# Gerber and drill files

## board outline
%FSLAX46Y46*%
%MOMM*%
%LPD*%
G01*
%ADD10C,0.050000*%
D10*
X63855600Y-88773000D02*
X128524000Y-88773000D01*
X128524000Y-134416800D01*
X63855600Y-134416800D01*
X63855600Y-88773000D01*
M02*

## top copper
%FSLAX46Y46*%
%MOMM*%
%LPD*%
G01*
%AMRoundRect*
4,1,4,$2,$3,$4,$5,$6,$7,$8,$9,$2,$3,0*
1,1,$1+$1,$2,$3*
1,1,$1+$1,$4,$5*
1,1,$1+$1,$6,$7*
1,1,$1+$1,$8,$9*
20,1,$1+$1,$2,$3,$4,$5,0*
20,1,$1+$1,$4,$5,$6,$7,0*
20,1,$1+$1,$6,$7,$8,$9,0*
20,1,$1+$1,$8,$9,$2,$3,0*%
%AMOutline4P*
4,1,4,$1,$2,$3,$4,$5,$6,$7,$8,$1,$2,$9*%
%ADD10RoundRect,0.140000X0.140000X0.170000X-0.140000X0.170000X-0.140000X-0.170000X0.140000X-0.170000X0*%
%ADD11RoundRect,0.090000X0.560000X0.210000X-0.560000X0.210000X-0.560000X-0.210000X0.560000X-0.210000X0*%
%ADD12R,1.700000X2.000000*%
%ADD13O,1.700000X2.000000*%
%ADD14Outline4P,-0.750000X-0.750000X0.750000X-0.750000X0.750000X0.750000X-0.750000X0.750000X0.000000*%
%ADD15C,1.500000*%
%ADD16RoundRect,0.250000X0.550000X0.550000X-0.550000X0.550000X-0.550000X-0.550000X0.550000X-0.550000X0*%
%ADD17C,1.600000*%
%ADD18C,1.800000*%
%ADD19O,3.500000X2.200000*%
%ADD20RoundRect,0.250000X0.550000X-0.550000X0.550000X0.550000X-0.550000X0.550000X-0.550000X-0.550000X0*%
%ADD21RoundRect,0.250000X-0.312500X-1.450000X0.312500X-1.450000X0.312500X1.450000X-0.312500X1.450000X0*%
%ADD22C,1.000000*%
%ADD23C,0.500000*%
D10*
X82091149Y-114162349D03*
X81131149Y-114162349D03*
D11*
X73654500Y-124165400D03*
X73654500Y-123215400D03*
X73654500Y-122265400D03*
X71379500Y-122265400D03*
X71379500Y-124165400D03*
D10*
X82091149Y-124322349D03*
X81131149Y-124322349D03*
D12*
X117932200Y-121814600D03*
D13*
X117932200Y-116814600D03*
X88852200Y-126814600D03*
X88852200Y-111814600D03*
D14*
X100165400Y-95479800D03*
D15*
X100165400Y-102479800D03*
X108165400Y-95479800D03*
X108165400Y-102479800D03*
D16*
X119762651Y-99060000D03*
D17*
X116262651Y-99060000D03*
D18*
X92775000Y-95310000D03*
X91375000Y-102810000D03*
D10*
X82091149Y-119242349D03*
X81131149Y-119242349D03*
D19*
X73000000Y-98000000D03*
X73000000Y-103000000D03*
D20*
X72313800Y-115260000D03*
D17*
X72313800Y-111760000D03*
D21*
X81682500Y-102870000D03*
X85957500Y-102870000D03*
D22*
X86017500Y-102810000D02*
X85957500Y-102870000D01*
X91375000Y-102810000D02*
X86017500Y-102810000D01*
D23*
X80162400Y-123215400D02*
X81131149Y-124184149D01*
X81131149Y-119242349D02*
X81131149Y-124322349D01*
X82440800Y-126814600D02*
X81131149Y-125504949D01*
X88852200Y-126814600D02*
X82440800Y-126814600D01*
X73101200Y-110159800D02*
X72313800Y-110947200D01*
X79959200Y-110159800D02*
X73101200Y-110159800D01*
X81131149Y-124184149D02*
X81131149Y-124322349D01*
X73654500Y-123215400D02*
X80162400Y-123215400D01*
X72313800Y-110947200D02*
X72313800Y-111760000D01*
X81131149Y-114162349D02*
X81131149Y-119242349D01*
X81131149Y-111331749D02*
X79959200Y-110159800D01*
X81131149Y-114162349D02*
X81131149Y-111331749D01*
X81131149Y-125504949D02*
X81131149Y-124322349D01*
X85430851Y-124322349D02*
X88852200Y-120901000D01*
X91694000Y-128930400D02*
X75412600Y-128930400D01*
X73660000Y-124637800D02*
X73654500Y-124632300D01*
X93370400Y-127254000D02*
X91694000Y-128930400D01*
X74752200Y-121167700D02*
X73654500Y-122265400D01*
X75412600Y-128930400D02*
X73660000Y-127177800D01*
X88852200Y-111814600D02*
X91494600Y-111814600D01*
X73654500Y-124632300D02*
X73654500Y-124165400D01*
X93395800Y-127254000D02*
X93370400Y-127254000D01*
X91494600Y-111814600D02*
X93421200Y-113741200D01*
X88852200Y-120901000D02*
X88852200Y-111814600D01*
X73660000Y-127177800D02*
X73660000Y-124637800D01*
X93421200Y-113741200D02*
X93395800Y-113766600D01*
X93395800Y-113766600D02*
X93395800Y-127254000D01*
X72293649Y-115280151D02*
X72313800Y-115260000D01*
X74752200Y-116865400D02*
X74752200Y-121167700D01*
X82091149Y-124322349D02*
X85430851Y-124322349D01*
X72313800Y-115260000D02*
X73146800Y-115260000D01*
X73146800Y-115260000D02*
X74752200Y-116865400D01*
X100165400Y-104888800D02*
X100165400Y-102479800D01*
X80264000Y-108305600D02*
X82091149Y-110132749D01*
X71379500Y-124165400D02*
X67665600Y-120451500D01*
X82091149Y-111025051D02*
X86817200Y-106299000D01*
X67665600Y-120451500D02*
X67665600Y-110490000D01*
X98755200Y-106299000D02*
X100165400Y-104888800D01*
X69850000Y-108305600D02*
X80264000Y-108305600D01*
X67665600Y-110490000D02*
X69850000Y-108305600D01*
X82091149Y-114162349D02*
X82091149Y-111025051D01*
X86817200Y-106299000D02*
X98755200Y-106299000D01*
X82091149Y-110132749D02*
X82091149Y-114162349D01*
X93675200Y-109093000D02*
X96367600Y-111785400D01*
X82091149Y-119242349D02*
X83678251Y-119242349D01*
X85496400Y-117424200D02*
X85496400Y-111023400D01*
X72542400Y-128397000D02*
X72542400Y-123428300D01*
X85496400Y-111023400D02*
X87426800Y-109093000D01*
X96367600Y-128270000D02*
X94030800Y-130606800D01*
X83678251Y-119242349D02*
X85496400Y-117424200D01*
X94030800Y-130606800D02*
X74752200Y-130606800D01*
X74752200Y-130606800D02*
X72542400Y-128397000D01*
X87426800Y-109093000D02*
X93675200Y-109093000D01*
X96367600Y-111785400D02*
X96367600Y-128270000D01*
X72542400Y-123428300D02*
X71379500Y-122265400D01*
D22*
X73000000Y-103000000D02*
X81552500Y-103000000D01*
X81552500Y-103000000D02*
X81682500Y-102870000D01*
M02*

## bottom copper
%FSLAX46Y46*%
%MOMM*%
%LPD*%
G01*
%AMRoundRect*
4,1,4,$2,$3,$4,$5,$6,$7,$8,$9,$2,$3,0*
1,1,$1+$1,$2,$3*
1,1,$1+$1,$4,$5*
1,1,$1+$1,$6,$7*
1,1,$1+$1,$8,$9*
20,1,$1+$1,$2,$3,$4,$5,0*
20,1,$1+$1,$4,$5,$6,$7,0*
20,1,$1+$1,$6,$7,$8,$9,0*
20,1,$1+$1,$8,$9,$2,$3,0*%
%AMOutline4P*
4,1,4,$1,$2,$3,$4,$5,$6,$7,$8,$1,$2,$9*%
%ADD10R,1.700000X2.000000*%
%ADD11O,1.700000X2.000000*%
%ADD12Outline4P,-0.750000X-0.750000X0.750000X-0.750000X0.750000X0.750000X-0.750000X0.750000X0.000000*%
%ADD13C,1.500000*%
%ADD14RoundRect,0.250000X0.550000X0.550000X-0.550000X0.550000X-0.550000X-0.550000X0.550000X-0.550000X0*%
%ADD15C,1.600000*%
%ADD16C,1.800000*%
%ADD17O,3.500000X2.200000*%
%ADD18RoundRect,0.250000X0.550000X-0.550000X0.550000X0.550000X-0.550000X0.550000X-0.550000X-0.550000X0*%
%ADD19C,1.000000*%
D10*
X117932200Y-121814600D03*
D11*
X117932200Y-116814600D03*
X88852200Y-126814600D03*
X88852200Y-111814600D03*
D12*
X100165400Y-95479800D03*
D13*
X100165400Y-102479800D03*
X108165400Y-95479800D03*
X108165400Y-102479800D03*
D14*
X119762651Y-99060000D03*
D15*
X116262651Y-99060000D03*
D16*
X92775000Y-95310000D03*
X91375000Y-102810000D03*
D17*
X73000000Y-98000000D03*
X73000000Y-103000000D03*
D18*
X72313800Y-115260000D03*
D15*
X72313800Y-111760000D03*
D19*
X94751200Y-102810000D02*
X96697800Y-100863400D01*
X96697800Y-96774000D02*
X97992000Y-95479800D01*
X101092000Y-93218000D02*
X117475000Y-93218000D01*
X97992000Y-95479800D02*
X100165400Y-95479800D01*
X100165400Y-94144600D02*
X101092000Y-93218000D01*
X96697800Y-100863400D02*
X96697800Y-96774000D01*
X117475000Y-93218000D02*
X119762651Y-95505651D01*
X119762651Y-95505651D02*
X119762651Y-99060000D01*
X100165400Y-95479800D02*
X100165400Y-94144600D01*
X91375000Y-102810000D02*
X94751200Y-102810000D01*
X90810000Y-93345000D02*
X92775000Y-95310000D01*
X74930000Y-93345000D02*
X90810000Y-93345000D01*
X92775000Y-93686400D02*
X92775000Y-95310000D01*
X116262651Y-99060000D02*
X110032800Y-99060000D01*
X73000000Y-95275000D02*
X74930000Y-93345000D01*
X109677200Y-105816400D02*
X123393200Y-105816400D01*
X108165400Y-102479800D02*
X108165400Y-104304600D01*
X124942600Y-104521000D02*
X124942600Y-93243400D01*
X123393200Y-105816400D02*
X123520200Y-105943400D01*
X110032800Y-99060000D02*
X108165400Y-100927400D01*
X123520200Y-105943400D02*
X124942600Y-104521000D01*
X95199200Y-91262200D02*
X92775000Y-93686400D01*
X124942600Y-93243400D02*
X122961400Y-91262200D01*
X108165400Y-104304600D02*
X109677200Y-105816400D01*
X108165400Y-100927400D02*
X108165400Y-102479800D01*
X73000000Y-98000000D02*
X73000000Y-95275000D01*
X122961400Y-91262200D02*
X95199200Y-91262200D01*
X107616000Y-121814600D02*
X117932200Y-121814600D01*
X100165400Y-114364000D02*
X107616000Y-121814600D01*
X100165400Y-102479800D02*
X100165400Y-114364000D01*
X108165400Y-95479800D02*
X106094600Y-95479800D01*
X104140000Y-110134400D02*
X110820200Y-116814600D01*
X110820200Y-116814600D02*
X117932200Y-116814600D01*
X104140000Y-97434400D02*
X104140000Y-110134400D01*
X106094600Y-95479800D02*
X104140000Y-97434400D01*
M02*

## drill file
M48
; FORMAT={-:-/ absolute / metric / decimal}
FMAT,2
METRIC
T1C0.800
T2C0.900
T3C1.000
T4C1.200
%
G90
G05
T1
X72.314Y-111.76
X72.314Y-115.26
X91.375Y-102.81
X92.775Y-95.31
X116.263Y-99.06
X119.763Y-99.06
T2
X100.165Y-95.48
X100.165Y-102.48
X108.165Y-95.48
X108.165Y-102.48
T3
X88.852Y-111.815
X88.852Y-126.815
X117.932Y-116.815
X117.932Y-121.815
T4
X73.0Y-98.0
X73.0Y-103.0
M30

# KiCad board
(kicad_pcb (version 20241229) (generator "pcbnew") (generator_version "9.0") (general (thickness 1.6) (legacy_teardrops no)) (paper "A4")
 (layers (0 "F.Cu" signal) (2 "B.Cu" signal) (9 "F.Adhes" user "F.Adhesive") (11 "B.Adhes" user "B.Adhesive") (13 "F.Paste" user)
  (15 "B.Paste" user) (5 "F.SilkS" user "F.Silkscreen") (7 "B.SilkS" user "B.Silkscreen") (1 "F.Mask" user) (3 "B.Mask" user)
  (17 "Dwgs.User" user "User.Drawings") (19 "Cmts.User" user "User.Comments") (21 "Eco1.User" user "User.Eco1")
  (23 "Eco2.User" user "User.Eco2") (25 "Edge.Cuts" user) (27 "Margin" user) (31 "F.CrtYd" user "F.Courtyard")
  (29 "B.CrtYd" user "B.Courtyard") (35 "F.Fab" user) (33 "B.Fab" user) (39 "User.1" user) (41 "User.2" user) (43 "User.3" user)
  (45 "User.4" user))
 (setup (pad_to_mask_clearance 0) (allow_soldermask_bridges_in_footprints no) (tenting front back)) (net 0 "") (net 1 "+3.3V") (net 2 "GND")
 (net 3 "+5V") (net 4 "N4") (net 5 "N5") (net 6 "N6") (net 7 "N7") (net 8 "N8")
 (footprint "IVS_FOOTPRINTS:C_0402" (layer "F.Cu") (at 81.611149 114.162349 180)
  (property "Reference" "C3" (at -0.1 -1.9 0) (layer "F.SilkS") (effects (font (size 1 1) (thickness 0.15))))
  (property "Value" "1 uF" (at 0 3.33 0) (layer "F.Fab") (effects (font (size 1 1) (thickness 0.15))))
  (pad "1" smd roundrect (at -0.48 0 180) (size 0.56 0.62) (layers "F.Cu" "F.Mask" "F.Paste") (roundrect_rratio 0.25) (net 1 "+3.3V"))
  (pad "2" smd roundrect (at 0.48 0 180) (size 0.56 0.62) (layers "F.Cu" "F.Mask" "F.Paste") (roundrect_rratio 0.25) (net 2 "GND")))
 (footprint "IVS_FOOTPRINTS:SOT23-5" (layer "F.Cu") (at 72.517 123.2154 180)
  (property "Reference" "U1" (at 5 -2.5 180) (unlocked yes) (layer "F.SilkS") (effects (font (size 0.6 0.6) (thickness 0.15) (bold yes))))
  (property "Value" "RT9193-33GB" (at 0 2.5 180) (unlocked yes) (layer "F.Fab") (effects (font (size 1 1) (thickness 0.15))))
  (pad "1" smd roundrect (at -1.1375 -0.95 180) (size 1.3 0.6) (layers "F.Cu" "F.Mask" "F.Paste") (roundrect_rratio 0.15) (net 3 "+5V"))
  (pad "2" smd roundrect (at -1.1375 0 180) (size 1.3 0.6) (layers "F.Cu" "F.Mask" "F.Paste") (roundrect_rratio 0.15) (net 2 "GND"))
  (pad "3" smd roundrect (at -1.1375 0.95 180) (size 1.3 0.6) (layers "F.Cu" "F.Mask" "F.Paste") (roundrect_rratio 0.15) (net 3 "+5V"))
  (pad "4" smd roundrect (at 1.1375 0.95 180) (size 1.3 0.6) (layers "F.Cu" "F.Mask" "F.Paste") (roundrect_rratio 0.15) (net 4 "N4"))
  (pad "5" smd roundrect (at 1.1375 -0.95 180) (size 1.3 0.6) (layers "F.Cu" "F.Mask" "F.Paste") (roundrect_rratio 0.15) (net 1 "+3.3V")))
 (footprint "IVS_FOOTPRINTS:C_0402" (layer "F.Cu") (at 81.611149 124.322349 180)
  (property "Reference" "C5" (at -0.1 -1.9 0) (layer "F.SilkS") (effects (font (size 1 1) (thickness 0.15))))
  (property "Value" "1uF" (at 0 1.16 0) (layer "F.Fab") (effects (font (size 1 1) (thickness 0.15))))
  (pad "1" smd roundrect (at -0.48 0 180) (size 0.56 0.62) (layers "F.Cu" "F.Mask" "F.Paste") (roundrect_rratio 0.25) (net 3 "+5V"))
  (pad "2" smd roundrect (at 0.48 0 180) (size 0.56 0.62) (layers "F.Cu" "F.Mask" "F.Paste") (roundrect_rratio 0.25) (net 2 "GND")))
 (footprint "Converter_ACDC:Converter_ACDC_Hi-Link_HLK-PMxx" (layer "F.Cu") (at 117.9322 121.8146 180)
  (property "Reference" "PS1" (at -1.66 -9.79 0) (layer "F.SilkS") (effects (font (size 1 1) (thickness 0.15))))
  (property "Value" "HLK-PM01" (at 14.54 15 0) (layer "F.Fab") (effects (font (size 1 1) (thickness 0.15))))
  (pad "1" thru_hole rect (at 0 0 180) (size 1.7 2) (drill 1) (layers "*.Cu" "*.Mask") (remove_unused_layers no) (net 1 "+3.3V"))
  (pad "2" thru_hole oval (at 0 5 180) (size 1.7 2) (drill 1) (layers "*.Cu" "*.Mask") (remove_unused_layers no) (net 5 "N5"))
  (pad "3" thru_hole oval (at 29.08 -5 180) (size 1.7 2) (drill 1) (layers "*.Cu" "*.Mask") (remove_unused_layers no) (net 2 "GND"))
  (pad "4" thru_hole oval (at 29.08 10 180) (size 1.7 2) (drill 1) (layers "*.Cu" "*.Mask") (remove_unused_layers no) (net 3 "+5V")))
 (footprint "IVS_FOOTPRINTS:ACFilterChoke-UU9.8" (layer "F.Cu") (at 104.1154 98.8798)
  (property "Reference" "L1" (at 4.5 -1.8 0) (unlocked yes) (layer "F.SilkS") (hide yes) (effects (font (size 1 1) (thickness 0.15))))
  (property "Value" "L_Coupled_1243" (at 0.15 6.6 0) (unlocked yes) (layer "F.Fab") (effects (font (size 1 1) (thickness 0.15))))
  (pad "1" thru_hole trapezoid (at -3.95 -3.4) (size 1.5 1.5) (drill 0.9) (layers "*.Cu" "*.Mask") (remove_unused_layers no) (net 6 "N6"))
  (pad "2" thru_hole circle (at -3.95 3.6) (size 1.5 1.5) (drill 0.9) (layers "*.Cu" "*.Mask") (remove_unused_layers no) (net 1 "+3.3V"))
  (pad "3" thru_hole circle (at 4.05 -3.4) (size 1.5 1.5) (drill 0.9) (layers "*.Cu" "*.Mask") (remove_unused_layers no) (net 5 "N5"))
  (pad "4" thru_hole circle (at 4.05 3.6) (size 1.5 1.5) (drill 0.9) (layers "*.Cu" "*.Mask") (remove_unused_layers no) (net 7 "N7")))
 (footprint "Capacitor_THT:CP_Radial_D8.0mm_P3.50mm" (layer "F.Cu") (at 119.762651 99.06 180)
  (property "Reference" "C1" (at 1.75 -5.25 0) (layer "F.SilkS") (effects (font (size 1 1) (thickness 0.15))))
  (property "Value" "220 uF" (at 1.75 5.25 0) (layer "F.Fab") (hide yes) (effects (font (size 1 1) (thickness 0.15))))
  (pad "1" thru_hole roundrect (at 0 0 180) (size 1.6 1.6) (drill 0.8) (layers "*.Cu" "*.Mask") (remove_unused_layers no)
   (roundrect_rratio 0.15625) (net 6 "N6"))
  (pad "2" thru_hole circle (at 3.5 0 180) (size 1.6 1.6) (drill 0.8) (layers "*.Cu" "*.Mask") (remove_unused_layers no) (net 7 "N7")))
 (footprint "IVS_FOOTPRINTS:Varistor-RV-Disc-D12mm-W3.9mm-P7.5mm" (layer "F.Cu") (at 92.775 95.31 -90)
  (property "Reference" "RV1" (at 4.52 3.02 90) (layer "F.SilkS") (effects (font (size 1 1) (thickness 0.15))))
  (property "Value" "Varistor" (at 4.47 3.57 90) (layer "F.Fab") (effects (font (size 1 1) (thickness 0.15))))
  (pad "1" thru_hole circle (at 0 0 270) (size 1.8 1.8) (drill 0.8) (layers "*.Cu" "*.Mask") (remove_unused_layers no) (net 7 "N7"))
  (pad "2" thru_hole circle (at 7.5 1.4 270) (size 1.8 1.8) (drill 0.8) (layers "*.Cu" "*.Mask") (remove_unused_layers no) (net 6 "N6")))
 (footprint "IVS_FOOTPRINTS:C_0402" (layer "F.Cu") (at 81.611149 119.242349 180)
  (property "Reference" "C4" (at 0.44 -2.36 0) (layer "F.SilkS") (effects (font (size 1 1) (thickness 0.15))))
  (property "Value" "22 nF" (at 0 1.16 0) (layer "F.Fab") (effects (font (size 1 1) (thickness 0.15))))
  (pad "1" smd roundrect (at -0.48 0 180) (size 0.56 0.62) (layers "F.Cu" "F.Mask" "F.Paste") (roundrect_rratio 0.25) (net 4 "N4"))
  (pad "2" smd roundrect (at 0.48 0 180) (size 0.56 0.62) (layers "F.Cu" "F.Mask" "F.Paste") (roundrect_rratio 0.25) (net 2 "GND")))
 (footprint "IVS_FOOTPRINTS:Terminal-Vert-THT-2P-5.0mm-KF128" (layer "F.Cu") (at 73 100.5 -90)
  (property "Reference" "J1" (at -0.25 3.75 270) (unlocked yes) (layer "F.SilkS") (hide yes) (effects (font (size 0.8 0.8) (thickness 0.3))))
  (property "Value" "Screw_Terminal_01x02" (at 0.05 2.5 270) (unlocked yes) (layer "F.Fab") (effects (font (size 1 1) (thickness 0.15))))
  (pad "1" thru_hole oval (at -2.5 0 270) (size 2.2 3.5) (drill 1.2) (layers "*.Cu" "*.Mask") (remove_unused_layers no) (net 7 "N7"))
  (pad "2" thru_hole oval (at 2.5 0 270) (size 2.2 3.5) (drill 1.2) (layers "*.Cu" "*.Mask") (remove_unused_layers no) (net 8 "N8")))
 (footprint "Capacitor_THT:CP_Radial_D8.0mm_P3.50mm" (layer "F.Cu") (at 72.3138 115.26 90)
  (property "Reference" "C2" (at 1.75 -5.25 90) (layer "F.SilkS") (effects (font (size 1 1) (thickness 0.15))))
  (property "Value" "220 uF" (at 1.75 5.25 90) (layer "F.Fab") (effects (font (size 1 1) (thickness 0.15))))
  (pad "1" thru_hole roundrect (at 0 0 90) (size 1.6 1.6) (drill 0.8) (layers "*.Cu" "*.Mask") (remove_unused_layers no)
   (roundrect_rratio 0.15625) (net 3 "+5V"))
  (pad "2" thru_hole circle (at 3.5 0 90) (size 1.6 1.6) (drill 0.8) (layers "*.Cu" "*.Mask") (remove_unused_layers no) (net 2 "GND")))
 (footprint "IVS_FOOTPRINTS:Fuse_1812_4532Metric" (layer "F.Cu") (at 83.82 102.87)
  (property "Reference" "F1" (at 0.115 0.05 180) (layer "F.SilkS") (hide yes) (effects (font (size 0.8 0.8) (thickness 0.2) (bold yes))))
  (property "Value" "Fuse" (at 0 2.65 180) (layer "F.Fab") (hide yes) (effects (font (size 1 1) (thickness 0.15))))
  (pad "1" smd roundrect (at -2.1375 0) (size 1.125 3.4) (layers "F.Cu" "F.Mask" "F.Paste") (roundrect_rratio 0.2222222222) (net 8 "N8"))
  (pad "2" smd roundrect (at 2.1375 0) (size 1.125 3.4) (layers "F.Cu" "F.Mask" "F.Paste") (roundrect_rratio 0.2222222222) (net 6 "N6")))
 (gr_rect (start 63.8556 88.773) (end 128.524 134.4168) (stroke (width 0.05) (type default)) (fill no) (layer "Edge.Cuts"))
 (segment (start 86.0175 102.81) (end 85.9575 102.87) (width 1) (layer "F.Cu") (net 6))
 (segment (start 91.375 102.81) (end 86.0175 102.81) (width 1) (layer "F.Cu") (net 6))
 (segment (start 94.7512 102.81) (end 96.6978 100.8634) (width 1) (layer "B.Cu") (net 6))
 (segment (start 96.6978 96.774) (end 97.992 95.4798) (width 1) (layer "B.Cu") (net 6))
 (segment (start 101.092 93.218) (end 117.475 93.218) (width 1) (layer "B.Cu") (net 6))
 (segment (start 97.992 95.4798) (end 100.1654 95.4798) (width 1) (layer "B.Cu") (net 6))
 (segment (start 100.1654 94.1446) (end 101.092 93.218) (width 1) (layer "B.Cu") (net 6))
 (segment (start 96.6978 100.8634) (end 96.6978 96.774) (width 1) (layer "B.Cu") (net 6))
 (segment (start 117.475 93.218) (end 119.762651 95.505651) (width 1) (layer "B.Cu") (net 6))
 (segment (start 119.762651 95.505651) (end 119.762651 99.06) (width 1) (layer "B.Cu") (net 6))
 (segment (start 100.1654 95.4798) (end 100.1654 94.1446) (width 1) (layer "B.Cu") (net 6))
 (segment (start 91.375 102.81) (end 94.7512 102.81) (width 1) (layer "B.Cu") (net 6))
 (segment (start 90.81 93.345) (end 92.775 95.31) (width 1) (layer "B.Cu") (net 7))
 (segment (start 74.93 93.345) (end 90.81 93.345) (width 1) (layer "B.Cu") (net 7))
 (segment (start 92.775 93.6864) (end 92.775 95.31) (width 1) (layer "B.Cu") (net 7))
 (segment (start 116.262651 99.06) (end 110.0328 99.06) (width 1) (layer "B.Cu") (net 7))
 (segment (start 73 95.275) (end 74.93 93.345) (width 1) (layer "B.Cu") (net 7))
 (segment (start 109.6772 105.8164) (end 123.3932 105.8164) (width 1) (layer "B.Cu") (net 7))
 (segment (start 108.1654 102.4798) (end 108.1654 104.3046) (width 1) (layer "B.Cu") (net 7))
 (segment (start 124.9426 104.521) (end 124.9426 93.2434) (width 1) (layer "B.Cu") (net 7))
 (segment (start 123.3932 105.8164) (end 123.5202 105.9434) (width 1) (layer "B.Cu") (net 7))
 (segment (start 110.0328 99.06) (end 108.1654 100.9274) (width 1) (layer "B.Cu") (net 7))
 (segment (start 123.5202 105.9434) (end 124.9426 104.521) (width 1) (layer "B.Cu") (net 7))
 (segment (start 95.1992 91.2622) (end 92.775 93.6864) (width 1) (layer "B.Cu") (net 7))
 (segment (start 124.9426 93.2434) (end 122.9614 91.2622) (width 1) (layer "B.Cu") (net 7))
 (segment (start 108.1654 104.3046) (end 109.6772 105.8164) (width 1) (layer "B.Cu") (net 7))
 (segment (start 108.1654 100.9274) (end 108.1654 102.4798) (width 1) (layer "B.Cu") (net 7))
 (segment (start 73 98) (end 73 95.275) (width 1) (layer "B.Cu") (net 7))
 (segment (start 122.9614 91.2622) (end 95.1992 91.2622) (width 1) (layer "B.Cu") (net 7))
 (segment (start 80.1624 123.2154) (end 81.131149 124.184149) (width 0.5) (layer "F.Cu") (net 2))
 (segment (start 81.131149 119.242349) (end 81.131149 124.322349) (width 0.5) (layer "F.Cu") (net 2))
 (segment (start 82.4408 126.8146) (end 81.131149 125.504949) (width 0.5) (layer "F.Cu") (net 2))
 (segment (start 88.8522 126.8146) (end 82.4408 126.8146) (width 0.5) (layer "F.Cu") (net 2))
 (segment (start 73.1012 110.1598) (end 72.3138 110.9472) (width 0.5) (layer "F.Cu") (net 2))
 (segment (start 79.9592 110.1598) (end 73.1012 110.1598) (width 0.5) (layer "F.Cu") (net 2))
 (segment (start 81.131149 124.184149) (end 81.131149 124.322349) (width 0.5) (layer "F.Cu") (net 2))
 (segment (start 73.6545 123.2154) (end 80.1624 123.2154) (width 0.5) (layer "F.Cu") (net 2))
 (segment (start 72.3138 110.9472) (end 72.3138 111.76) (width 0.5) (layer "F.Cu") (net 2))
 (segment (start 81.131149 114.162349) (end 81.131149 119.242349) (width 0.5) (layer "F.Cu") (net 2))
 (segment (start 81.131149 111.331749) (end 79.9592 110.1598) (width 0.5) (layer "F.Cu") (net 2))
 (segment (start 81.131149 114.162349) (end 81.131149 111.331749) (width 0.5) (layer "F.Cu") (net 2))
 (segment (start 81.131149 125.504949) (end 81.131149 124.322349) (width 0.5) (layer "F.Cu") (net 2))
 (segment (start 85.430851 124.322349) (end 88.8522 120.901) (width 0.5) (layer "F.Cu") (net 3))
 (segment (start 91.694 128.9304) (end 75.4126 128.9304) (width 0.5) (layer "F.Cu") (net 3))
 (segment (start 73.66 124.6378) (end 73.6545 124.6323) (width 0.5) (layer "F.Cu") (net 3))
 (segment (start 93.3704 127.254) (end 91.694 128.9304) (width 0.5) (layer "F.Cu") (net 3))
 (segment (start 74.7522 121.1677) (end 73.6545 122.2654) (width 0.5) (layer "F.Cu") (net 3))
 (segment (start 75.4126 128.9304) (end 73.66 127.1778) (width 0.5) (layer "F.Cu") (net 3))
 (segment (start 88.8522 111.8146) (end 91.4946 111.8146) (width 0.5) (layer "F.Cu") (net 3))
 (segment (start 73.6545 124.6323) (end 73.6545 124.1654) (width 0.5) (layer "F.Cu") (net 3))
 (segment (start 93.3958 127.254) (end 93.3704 127.254) (width 0.5) (layer "F.Cu") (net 3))
 (segment (start 91.4946 111.8146) (end 93.4212 113.7412) (width 0.5) (layer "F.Cu") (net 3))
 (segment (start 88.8522 120.901) (end 88.8522 111.8146) (width 0.5) (layer "F.Cu") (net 3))
 (segment (start 73.66 127.1778) (end 73.66 124.6378) (width 0.5) (layer "F.Cu") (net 3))
 (segment (start 93.4212 113.7412) (end 93.3958 113.7666) (width 0.5) (layer "F.Cu") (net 3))
 (segment (start 93.3958 113.7666) (end 93.3958 127.254) (width 0.5) (layer "F.Cu") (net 3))
 (segment (start 72.293649 115.280151) (end 72.3138 115.26) (width 0.5) (layer "F.Cu") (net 3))
 (segment (start 74.7522 116.8654) (end 74.7522 121.1677) (width 0.5) (layer "F.Cu") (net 3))
 (segment (start 82.091149 124.322349) (end 85.430851 124.322349) (width 0.5) (layer "F.Cu") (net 3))
 (segment (start 72.3138 115.26) (end 73.1468 115.26) (width 0.5) (layer "F.Cu") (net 3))
 (segment (start 73.1468 115.26) (end 74.7522 116.8654) (width 0.5) (layer "F.Cu") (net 3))
 (segment (start 100.1654 104.8888) (end 100.1654 102.4798) (width 0.5) (layer "F.Cu") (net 1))
 (segment (start 80.264 108.3056) (end 82.091149 110.132749) (width 0.5) (layer "F.Cu") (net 1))
 (segment (start 71.3795 124.1654) (end 67.6656 120.4515) (width 0.5) (layer "F.Cu") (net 1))
 (segment (start 82.091149 111.025051) (end 86.8172 106.299) (width 0.5) (layer "F.Cu") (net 1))
 (segment (start 67.6656 120.4515) (end 67.6656 110.49) (width 0.5) (layer "F.Cu") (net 1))
 (segment (start 98.7552 106.299) (end 100.1654 104.8888) (width 0.5) (layer "F.Cu") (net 1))
 (segment (start 69.85 108.3056) (end 80.264 108.3056) (width 0.5) (layer "F.Cu") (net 1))
 (segment (start 67.6656 110.49) (end 69.85 108.3056) (width 0.5) (layer "F.Cu") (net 1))
 (segment (start 82.091149 114.162349) (end 82.091149 111.025051) (width 0.5) (layer "F.Cu") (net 1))
 (segment (start 86.8172 106.299) (end 98.7552 106.299) (width 0.5) (layer "F.Cu") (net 1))
 (segment (start 82.091149 110.132749) (end 82.091149 114.162349) (width 0.5) (layer "F.Cu") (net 1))
 (segment (start 107.616 121.8146) (end 117.9322 121.8146) (width 1) (layer "B.Cu") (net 1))
 (segment (start 100.1654 114.364) (end 107.616 121.8146) (width 1) (layer "B.Cu") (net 1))
 (segment (start 100.1654 102.4798) (end 100.1654 114.364) (width 1) (layer "B.Cu") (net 1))
 (segment (start 93.6752 109.093) (end 96.3676 111.7854) (width 0.5) (layer "F.Cu") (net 4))
 (segment (start 82.091149 119.242349) (end 83.678251 119.242349) (width 0.5) (layer "F.Cu") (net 4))
 (segment (start 85.4964 117.4242) (end 85.4964 111.0234) (width 0.5) (layer "F.Cu") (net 4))
 (segment (start 72.5424 128.397) (end 72.5424 123.4283) (width 0.5) (layer "F.Cu") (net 4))
 (segment (start 85.4964 111.0234) (end 87.4268 109.093) (width 0.5) (layer "F.Cu") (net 4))
 (segment (start 96.3676 128.27) (end 94.0308 130.6068) (width 0.5) (layer "F.Cu") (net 4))
 (segment (start 83.678251 119.242349) (end 85.4964 117.4242) (width 0.5) (layer "F.Cu") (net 4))
 (segment (start 94.0308 130.6068) (end 74.7522 130.6068) (width 0.5) (layer "F.Cu") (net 4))
 (segment (start 74.7522 130.6068) (end 72.5424 128.397) (width 0.5) (layer "F.Cu") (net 4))
 (segment (start 87.4268 109.093) (end 93.6752 109.093) (width 0.5) (layer "F.Cu") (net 4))
 (segment (start 96.3676 111.7854) (end 96.3676 128.27) (width 0.5) (layer "F.Cu") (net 4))
 (segment (start 72.5424 123.4283) (end 71.3795 122.2654) (width 0.5) (layer "F.Cu") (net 4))
 (segment (start 73 103) (end 81.5525 103) (width 1) (layer "F.Cu") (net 8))
 (segment (start 81.5525 103) (end 81.6825 102.87) (width 1) (layer "F.Cu") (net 8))
 (segment (start 108.1654 95.4798) (end 106.0946 95.4798) (width 1) (layer "B.Cu") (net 5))
 (segment (start 104.14 110.1344) (end 110.8202 116.8146) (width 1) (layer "B.Cu") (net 5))
 (segment (start 110.8202 116.8146) (end 117.9322 116.8146) (width 1) (layer "B.Cu") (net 5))
 (segment (start 104.14 97.4344) (end 104.14 110.1344) (width 1) (layer "B.Cu") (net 5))
 (segment (start 106.0946 95.4798) (end 104.14 97.4344) (width 1) (layer "B.Cu") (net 5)))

